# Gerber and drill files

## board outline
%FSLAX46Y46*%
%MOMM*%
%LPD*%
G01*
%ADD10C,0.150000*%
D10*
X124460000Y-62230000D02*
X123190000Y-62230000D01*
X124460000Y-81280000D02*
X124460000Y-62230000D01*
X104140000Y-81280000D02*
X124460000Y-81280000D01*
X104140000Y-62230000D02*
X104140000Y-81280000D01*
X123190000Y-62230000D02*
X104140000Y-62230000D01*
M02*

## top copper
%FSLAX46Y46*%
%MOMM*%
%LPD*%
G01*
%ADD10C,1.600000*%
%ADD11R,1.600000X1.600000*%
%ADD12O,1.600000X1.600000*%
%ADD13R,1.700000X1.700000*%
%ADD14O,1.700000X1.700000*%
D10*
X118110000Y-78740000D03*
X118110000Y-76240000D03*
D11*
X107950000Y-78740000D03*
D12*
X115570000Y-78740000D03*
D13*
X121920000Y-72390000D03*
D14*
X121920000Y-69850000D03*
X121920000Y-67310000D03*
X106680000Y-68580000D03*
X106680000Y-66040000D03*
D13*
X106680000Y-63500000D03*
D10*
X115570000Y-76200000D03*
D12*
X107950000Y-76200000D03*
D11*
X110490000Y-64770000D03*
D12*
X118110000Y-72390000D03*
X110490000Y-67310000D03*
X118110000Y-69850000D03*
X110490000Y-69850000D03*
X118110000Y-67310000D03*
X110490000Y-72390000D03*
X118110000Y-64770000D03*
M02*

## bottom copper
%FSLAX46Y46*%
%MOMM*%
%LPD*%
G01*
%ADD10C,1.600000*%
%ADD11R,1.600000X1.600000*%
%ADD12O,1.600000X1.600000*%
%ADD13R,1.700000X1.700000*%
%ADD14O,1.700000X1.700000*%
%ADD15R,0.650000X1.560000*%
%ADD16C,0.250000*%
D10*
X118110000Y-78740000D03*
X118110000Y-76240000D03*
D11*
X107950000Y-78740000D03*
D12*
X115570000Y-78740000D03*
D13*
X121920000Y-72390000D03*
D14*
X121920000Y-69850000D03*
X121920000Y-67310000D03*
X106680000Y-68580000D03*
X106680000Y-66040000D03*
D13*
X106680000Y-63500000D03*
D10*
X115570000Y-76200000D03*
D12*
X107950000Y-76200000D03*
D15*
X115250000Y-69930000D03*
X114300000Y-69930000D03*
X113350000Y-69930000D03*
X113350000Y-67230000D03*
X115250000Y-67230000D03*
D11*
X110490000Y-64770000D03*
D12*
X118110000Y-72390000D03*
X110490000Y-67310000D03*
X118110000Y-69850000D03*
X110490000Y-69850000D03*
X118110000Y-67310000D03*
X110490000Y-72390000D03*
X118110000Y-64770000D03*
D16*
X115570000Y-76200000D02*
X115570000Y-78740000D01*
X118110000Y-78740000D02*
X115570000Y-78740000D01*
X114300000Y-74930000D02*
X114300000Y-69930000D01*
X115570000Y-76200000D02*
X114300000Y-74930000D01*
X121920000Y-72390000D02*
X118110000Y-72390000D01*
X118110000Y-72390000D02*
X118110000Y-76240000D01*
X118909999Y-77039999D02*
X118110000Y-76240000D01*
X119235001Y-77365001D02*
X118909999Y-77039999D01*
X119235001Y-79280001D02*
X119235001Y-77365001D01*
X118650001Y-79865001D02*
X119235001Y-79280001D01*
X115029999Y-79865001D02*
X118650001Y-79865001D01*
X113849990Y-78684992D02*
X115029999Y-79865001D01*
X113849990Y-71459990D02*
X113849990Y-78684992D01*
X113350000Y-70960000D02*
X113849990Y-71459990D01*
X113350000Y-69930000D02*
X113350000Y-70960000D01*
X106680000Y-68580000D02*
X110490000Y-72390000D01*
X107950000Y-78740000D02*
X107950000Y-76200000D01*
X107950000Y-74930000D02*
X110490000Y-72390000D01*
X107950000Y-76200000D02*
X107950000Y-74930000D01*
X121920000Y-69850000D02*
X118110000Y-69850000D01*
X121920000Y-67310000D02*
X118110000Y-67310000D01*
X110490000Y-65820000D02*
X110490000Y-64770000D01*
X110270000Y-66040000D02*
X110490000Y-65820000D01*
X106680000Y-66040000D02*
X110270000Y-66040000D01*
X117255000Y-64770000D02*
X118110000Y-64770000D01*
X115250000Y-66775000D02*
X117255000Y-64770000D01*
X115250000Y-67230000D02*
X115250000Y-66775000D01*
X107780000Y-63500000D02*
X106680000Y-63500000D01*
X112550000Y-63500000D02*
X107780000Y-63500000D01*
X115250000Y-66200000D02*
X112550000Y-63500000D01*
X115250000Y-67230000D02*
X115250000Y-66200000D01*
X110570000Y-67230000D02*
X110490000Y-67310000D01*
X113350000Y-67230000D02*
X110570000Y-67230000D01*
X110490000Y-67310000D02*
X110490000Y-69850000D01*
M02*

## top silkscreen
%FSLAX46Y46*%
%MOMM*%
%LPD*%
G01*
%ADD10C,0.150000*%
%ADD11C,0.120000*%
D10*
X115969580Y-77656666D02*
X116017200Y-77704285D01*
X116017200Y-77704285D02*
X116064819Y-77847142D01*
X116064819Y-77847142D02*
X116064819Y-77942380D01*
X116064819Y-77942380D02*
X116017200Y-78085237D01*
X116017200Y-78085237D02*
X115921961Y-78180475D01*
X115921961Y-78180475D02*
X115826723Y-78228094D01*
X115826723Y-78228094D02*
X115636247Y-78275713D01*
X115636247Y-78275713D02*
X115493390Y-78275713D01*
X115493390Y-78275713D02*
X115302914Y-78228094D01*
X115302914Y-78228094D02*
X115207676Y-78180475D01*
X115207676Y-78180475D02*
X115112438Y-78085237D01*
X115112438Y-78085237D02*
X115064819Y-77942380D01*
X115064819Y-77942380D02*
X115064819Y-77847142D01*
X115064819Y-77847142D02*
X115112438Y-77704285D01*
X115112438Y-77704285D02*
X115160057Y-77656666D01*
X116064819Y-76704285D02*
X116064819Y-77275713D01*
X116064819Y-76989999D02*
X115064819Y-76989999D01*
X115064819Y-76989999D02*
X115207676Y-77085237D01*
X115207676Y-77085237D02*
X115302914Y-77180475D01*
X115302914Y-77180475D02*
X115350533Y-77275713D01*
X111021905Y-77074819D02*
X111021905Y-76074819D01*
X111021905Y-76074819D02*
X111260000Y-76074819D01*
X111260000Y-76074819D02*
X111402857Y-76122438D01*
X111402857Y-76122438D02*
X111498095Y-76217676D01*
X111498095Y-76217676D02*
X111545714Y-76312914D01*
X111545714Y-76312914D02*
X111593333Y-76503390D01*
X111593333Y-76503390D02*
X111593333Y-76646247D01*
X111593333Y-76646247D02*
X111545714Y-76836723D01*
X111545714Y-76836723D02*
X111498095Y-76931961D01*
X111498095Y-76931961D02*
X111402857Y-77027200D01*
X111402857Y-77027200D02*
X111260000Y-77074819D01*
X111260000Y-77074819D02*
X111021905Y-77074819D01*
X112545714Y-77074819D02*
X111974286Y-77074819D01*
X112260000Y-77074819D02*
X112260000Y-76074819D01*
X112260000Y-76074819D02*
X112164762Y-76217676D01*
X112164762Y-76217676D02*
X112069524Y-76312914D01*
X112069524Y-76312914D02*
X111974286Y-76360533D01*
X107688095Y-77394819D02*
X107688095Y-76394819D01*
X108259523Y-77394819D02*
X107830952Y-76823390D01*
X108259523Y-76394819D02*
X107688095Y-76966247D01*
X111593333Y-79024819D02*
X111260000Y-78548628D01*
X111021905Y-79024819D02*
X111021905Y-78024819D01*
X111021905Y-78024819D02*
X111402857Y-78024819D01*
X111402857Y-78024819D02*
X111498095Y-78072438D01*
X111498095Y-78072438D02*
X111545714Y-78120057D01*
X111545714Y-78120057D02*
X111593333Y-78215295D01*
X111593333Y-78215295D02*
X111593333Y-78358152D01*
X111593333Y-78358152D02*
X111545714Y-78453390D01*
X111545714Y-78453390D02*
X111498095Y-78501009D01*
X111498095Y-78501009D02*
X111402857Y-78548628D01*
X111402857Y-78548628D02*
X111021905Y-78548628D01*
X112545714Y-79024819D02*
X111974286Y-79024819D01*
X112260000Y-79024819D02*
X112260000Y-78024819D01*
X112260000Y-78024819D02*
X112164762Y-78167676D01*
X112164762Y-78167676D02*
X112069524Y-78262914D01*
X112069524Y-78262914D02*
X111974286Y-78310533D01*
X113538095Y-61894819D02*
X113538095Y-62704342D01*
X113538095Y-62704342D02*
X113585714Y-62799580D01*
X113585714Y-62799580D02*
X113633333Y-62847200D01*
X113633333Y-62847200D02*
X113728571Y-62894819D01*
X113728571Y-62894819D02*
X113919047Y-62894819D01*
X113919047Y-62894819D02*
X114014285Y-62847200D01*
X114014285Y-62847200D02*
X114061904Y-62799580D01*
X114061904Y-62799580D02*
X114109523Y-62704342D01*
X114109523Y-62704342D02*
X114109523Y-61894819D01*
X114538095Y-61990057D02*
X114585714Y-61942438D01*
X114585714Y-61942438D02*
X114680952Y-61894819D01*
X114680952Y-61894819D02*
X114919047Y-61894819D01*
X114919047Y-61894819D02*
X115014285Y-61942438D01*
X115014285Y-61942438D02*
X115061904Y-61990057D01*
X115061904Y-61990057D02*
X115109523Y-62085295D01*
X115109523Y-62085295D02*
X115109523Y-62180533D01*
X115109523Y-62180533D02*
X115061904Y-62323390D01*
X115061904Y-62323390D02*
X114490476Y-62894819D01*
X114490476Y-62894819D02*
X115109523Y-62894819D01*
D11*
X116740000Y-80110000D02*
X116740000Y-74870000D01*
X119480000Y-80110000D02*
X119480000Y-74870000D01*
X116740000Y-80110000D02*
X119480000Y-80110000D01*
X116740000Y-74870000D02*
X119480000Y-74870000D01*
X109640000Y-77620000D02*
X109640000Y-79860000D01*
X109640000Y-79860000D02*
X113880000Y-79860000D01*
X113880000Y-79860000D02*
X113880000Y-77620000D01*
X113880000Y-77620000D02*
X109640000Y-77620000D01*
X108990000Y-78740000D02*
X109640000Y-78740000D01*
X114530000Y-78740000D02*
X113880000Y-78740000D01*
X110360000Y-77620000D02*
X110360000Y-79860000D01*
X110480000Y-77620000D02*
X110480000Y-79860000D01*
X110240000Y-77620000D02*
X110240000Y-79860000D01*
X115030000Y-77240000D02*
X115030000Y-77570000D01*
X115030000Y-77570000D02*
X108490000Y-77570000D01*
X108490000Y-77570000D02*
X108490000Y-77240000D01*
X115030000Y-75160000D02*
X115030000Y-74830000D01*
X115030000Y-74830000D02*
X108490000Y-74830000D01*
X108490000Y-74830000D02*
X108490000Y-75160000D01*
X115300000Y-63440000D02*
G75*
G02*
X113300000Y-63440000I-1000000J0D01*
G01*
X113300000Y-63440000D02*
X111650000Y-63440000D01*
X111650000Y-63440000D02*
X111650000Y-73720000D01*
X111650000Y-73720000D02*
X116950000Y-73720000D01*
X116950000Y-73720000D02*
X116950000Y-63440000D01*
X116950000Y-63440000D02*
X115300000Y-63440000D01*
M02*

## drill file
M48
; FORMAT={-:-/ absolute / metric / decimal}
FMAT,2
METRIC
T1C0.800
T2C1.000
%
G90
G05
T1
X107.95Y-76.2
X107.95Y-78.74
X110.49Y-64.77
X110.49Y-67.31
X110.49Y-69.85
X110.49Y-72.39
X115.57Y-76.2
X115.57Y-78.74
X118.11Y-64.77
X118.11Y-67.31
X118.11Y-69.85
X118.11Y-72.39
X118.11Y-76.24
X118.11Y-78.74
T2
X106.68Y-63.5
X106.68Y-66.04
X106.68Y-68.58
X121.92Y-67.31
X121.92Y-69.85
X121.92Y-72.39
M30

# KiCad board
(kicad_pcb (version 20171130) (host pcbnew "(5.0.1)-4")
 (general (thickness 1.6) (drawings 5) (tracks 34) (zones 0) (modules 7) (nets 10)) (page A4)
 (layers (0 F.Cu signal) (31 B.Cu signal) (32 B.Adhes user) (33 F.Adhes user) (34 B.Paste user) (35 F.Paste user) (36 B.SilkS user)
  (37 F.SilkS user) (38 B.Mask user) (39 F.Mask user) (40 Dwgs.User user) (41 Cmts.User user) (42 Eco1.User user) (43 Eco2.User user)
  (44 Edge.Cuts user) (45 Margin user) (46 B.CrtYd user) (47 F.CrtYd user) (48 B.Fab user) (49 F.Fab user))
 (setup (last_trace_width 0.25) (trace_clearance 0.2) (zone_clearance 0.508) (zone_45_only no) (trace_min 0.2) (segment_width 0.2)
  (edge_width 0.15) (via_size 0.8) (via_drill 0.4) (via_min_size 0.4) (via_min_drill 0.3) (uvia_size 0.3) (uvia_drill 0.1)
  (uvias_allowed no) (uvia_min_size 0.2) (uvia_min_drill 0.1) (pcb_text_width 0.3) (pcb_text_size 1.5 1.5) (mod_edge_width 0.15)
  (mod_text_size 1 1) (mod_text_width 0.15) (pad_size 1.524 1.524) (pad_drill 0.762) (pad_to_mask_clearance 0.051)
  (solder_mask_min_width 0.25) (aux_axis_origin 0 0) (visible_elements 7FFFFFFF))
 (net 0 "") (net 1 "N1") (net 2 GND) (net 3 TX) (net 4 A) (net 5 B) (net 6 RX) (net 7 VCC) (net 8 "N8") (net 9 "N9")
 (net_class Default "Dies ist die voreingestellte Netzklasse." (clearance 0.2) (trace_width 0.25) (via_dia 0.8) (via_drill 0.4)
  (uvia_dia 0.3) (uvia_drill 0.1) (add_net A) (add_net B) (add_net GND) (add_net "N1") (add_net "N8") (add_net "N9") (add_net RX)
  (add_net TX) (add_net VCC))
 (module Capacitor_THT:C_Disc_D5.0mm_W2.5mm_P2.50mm (layer F.Cu) (at 118.11 78.74 90)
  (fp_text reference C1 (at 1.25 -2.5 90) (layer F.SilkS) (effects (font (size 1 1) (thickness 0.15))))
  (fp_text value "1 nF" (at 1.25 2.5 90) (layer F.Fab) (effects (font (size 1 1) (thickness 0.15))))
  (fp_line (start -1.37 -1.37) (end 3.87 -1.37) (layer F.SilkS) (width 0.12))
  (fp_line (start -1.37 1.37) (end 3.87 1.37) (layer F.SilkS) (width 0.12))
  (fp_line (start -1.37 -1.37) (end -1.37 1.37) (layer F.SilkS) (width 0.12))
  (fp_line (start 3.87 -1.37) (end 3.87 1.37) (layer F.SilkS) (width 0.12))
  (pad 1 thru_hole circle (at 0 0 90) (size 1.6 1.6) (drill 0.8) (layers *.Cu *.Mask) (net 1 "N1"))
  (pad 2 thru_hole circle (at 2.5 0 90) (size 1.6 1.6) (drill 0.8) (layers *.Cu *.Mask) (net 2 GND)))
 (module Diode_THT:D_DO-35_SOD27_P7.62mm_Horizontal (layer F.Cu) (at 107.95 78.74)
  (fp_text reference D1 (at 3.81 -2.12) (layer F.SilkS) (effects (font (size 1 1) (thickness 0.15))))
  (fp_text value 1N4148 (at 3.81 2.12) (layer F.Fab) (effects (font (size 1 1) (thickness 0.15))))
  (fp_line (start 1.69 -1.12) (end 1.69 1.12) (layer F.SilkS) (width 0.12))
  (fp_line (start 1.69 1.12) (end 5.93 1.12) (layer F.SilkS) (width 0.12))
  (fp_line (start 5.93 1.12) (end 5.93 -1.12) (layer F.SilkS) (width 0.12))
  (fp_line (start 5.93 -1.12) (end 1.69 -1.12) (layer F.SilkS) (width 0.12))
  (fp_line (start 1.04 0) (end 1.69 0) (layer F.SilkS) (width 0.12))
  (fp_line (start 6.58 0) (end 5.93 0) (layer F.SilkS) (width 0.12))
  (fp_line (start 2.41 -1.12) (end 2.41 1.12) (layer F.SilkS) (width 0.12))
  (fp_line (start 2.53 -1.12) (end 2.53 1.12) (layer F.SilkS) (width 0.12))
  (fp_line (start 2.29 -1.12) (end 2.29 1.12) (layer F.SilkS) (width 0.12))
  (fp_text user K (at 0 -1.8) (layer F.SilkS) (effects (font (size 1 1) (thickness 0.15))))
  (pad 1 thru_hole rect (at 0 0) (size 1.6 1.6) (drill 0.8) (layers *.Cu *.Mask) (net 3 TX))
  (pad 2 thru_hole oval (at 7.62 0) (size 1.6 1.6) (drill 0.8) (layers *.Cu *.Mask) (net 1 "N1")))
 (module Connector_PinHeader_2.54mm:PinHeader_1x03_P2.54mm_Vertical (layer B.Cu) (at 121.92 72.39)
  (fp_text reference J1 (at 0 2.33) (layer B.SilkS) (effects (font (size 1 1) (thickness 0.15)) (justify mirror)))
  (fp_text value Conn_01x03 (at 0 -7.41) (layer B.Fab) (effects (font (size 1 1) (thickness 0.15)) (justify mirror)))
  (pad 1 thru_hole rect (at 0 0) (size 1.7 1.7) (drill 1) (layers *.Cu *.Mask) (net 2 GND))
  (pad 2 thru_hole oval (at 0 -2.54) (size 1.7 1.7) (drill 1) (layers *.Cu *.Mask) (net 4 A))
  (pad 3 thru_hole oval (at 0 -5.08) (size 1.7 1.7) (drill 1) (layers *.Cu *.Mask) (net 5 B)))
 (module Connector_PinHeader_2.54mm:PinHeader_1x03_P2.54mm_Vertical (layer B.Cu) (at 106.68 63.5 180)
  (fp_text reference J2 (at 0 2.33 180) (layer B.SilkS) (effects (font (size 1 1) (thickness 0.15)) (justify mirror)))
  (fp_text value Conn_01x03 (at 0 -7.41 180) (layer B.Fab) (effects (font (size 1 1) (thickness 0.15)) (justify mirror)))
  (pad 3 thru_hole oval (at 0 -5.08 180) (size 1.7 1.7) (drill 1) (layers *.Cu *.Mask) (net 3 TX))
  (pad 2 thru_hole oval (at 0 -2.54 180) (size 1.7 1.7) (drill 1) (layers *.Cu *.Mask) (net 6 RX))
  (pad 1 thru_hole rect (at 0 0 180) (size 1.7 1.7) (drill 1) (layers *.Cu *.Mask) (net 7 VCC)))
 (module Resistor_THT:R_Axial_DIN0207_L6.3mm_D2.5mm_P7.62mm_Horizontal (layer F.Cu) (at 115.57 76.2 180)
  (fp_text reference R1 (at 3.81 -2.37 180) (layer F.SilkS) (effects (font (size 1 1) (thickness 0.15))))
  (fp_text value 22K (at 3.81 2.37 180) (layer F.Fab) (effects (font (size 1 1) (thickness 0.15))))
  (fp_line (start 0.54 -1.04) (end 0.54 -1.37) (layer F.SilkS) (width 0.12))
  (fp_line (start 0.54 -1.37) (end 7.08 -1.37) (layer F.SilkS) (width 0.12))
  (fp_line (start 7.08 -1.37) (end 7.08 -1.04) (layer F.SilkS) (width 0.12))
  (fp_line (start 0.54 1.04) (end 0.54 1.37) (layer F.SilkS) (width 0.12))
  (fp_line (start 0.54 1.37) (end 7.08 1.37) (layer F.SilkS) (width 0.12))
  (fp_line (start 7.08 1.37) (end 7.08 1.04) (layer F.SilkS) (width 0.12))
  (pad 1 thru_hole circle (at 0 0 180) (size 1.6 1.6) (drill 0.8) (layers *.Cu *.Mask) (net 1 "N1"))
  (pad 2 thru_hole oval (at 7.62 0 180) (size 1.6 1.6) (drill 0.8) (layers *.Cu *.Mask) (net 3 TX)))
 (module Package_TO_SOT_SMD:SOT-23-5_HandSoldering (layer B.Cu) (at 114.3 68.58 90)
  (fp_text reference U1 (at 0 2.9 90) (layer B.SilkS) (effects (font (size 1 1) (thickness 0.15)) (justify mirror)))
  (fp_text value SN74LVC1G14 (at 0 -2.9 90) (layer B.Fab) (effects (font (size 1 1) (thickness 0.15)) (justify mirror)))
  (pad 1 smd rect (at -1.35 0.95 90) (size 1.56 0.65) (layers B.Cu B.Paste B.Mask) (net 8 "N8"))
  (pad 2 smd rect (at -1.35 0 90) (size 1.56 0.65) (layers B.Cu B.Paste B.Mask) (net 1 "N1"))
  (pad 3 smd rect (at -1.35 -0.95 90) (size 1.56 0.65) (layers B.Cu B.Paste B.Mask) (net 2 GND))
  (pad 4 smd rect (at 1.35 -0.95 90) (size 1.56 0.65) (layers B.Cu B.Paste B.Mask) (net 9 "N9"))
  (pad 5 smd rect (at 1.35 0.95 90) (size 1.56 0.65) (layers B.Cu B.Paste B.Mask) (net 7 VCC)))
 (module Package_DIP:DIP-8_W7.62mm (layer F.Cu) (at 110.49 64.77)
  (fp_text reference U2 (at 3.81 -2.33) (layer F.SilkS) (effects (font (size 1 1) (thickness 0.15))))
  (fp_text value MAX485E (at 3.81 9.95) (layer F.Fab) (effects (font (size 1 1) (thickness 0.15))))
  (fp_arc (start 3.81 -1.33) (end 2.81 -1.33) (angle -180) (layer F.SilkS) (width 0.12))
  (fp_line (start 2.81 -1.33) (end 1.16 -1.33) (layer F.SilkS) (width 0.12))
  (fp_line (start 1.16 -1.33) (end 1.16 8.95) (layer F.SilkS) (width 0.12))
  (fp_line (start 1.16 8.95) (end 6.46 8.95) (layer F.SilkS) (width 0.12))
  (fp_line (start 6.46 8.95) (end 6.46 -1.33) (layer F.SilkS) (width 0.12))
  (fp_line (start 6.46 -1.33) (end 4.81 -1.33) (layer F.SilkS) (width 0.12))
  (pad 1 thru_hole rect (at 0 0) (size 1.6 1.6) (drill 0.8) (layers *.Cu *.Mask) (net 6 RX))
  (pad 5 thru_hole oval (at 7.62 7.62) (size 1.6 1.6) (drill 0.8) (layers *.Cu *.Mask) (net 2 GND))
  (pad 2 thru_hole oval (at 0 2.54) (size 1.6 1.6) (drill 0.8) (layers *.Cu *.Mask) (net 9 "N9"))
  (pad 6 thru_hole oval (at 7.62 5.08) (size 1.6 1.6) (drill 0.8) (layers *.Cu *.Mask) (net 4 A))
  (pad 3 thru_hole oval (at 0 5.08) (size 1.6 1.6) (drill 0.8) (layers *.Cu *.Mask) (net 9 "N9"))
  (pad 7 thru_hole oval (at 7.62 2.54) (size 1.6 1.6) (drill 0.8) (layers *.Cu *.Mask) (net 5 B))
  (pad 4 thru_hole oval (at 0 7.62) (size 1.6 1.6) (drill 0.8) (layers *.Cu *.Mask) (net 3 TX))
  (pad 8 thru_hole oval (at 7.62 0) (size 1.6 1.6) (drill 0.8) (layers *.Cu *.Mask) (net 7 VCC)))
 (gr_line (start 124.46 62.23) (end 123.19 62.23) (layer Edge.Cuts) (width 0.15))
 (gr_line (start 124.46 81.28) (end 124.46 62.23) (layer Edge.Cuts) (width 0.15))
 (gr_line (start 104.14 81.28) (end 124.46 81.28) (layer Edge.Cuts) (width 0.15))
 (gr_line (start 104.14 62.23) (end 104.14 81.28) (layer Edge.Cuts) (width 0.15))
 (gr_line (start 123.19 62.23) (end 104.14 62.23) (layer Edge.Cuts) (width 0.15))
 (segment (start 115.57 76.2) (end 115.57 78.74) (width 0.25) (layer B.Cu) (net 1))
 (segment (start 118.11 78.74) (end 115.57 78.74) (width 0.25) (layer B.Cu) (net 1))
 (segment (start 114.3 74.93) (end 114.3 69.93) (width 0.25) (layer B.Cu) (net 1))
 (segment (start 115.57 76.2) (end 114.3 74.93) (width 0.25) (layer B.Cu) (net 1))
 (segment (start 121.92 72.39) (end 118.11 72.39) (width 0.25) (layer B.Cu) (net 2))
 (segment (start 118.11 72.39) (end 118.11 76.24) (width 0.25) (layer B.Cu) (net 2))
 (segment (start 118.909999 77.039999) (end 118.11 76.24) (width 0.25) (layer B.Cu) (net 2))
 (segment (start 119.235001 77.365001) (end 118.909999 77.039999) (width 0.25) (layer B.Cu) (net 2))
 (segment (start 119.235001 79.280001) (end 119.235001 77.365001) (width 0.25) (layer B.Cu) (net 2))
 (segment (start 118.650001 79.865001) (end 119.235001 79.280001) (width 0.25) (layer B.Cu) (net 2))
 (segment (start 115.029999 79.865001) (end 118.650001 79.865001) (width 0.25) (layer B.Cu) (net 2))
 (segment (start 113.84999 78.684992) (end 115.029999 79.865001) (width 0.25) (layer B.Cu) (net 2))
 (segment (start 113.84999 71.45999) (end 113.84999 78.684992) (width 0.25) (layer B.Cu) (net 2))
 (segment (start 113.35 70.96) (end 113.84999 71.45999) (width 0.25) (layer B.Cu) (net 2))
 (segment (start 113.35 69.93) (end 113.35 70.96) (width 0.25) (layer B.Cu) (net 2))
 (segment (start 106.68 68.58) (end 110.49 72.39) (width 0.25) (layer B.Cu) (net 3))
 (segment (start 107.95 78.74) (end 107.95 76.2) (width 0.25) (layer B.Cu) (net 3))
 (segment (start 107.95 74.93) (end 110.49 72.39) (width 0.25) (layer B.Cu) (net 3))
 (segment (start 107.95 76.2) (end 107.95 74.93) (width 0.25) (layer B.Cu) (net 3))
 (segment (start 121.92 69.85) (end 118.11 69.85) (width 0.25) (layer B.Cu) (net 4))
 (segment (start 121.92 67.31) (end 118.11 67.31) (width 0.25) (layer B.Cu) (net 5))
 (segment (start 110.49 65.82) (end 110.49 64.77) (width 0.25) (layer B.Cu) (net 6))
 (segment (start 110.27 66.04) (end 110.49 65.82) (width 0.25) (layer B.Cu) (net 6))
 (segment (start 106.68 66.04) (end 110.27 66.04) (width 0.25) (layer B.Cu) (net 6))
 (segment (start 117.255 64.77) (end 118.11 64.77) (width 0.25) (layer B.Cu) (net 7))
 (segment (start 115.25 66.775) (end 117.255 64.77) (width 0.25) (layer B.Cu) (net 7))
 (segment (start 115.25 67.23) (end 115.25 66.775) (width 0.25) (layer B.Cu) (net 7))
 (segment (start 107.78 63.5) (end 106.68 63.5) (width 0.25) (layer B.Cu) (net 7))
 (segment (start 112.55 63.5) (end 107.78 63.5) (width 0.25) (layer B.Cu) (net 7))
 (segment (start 115.25 66.2) (end 112.55 63.5) (width 0.25) (layer B.Cu) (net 7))
 (segment (start 115.25 67.23) (end 115.25 66.2) (width 0.25) (layer B.Cu) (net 7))
 (segment (start 110.57 67.23) (end 110.49 67.31) (width 0.25) (layer B.Cu) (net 9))
 (segment (start 113.35 67.23) (end 110.57 67.23) (width 0.25) (layer B.Cu) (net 9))
 (segment (start 110.49 67.31) (end 110.49 69.85) (width 0.25) (layer B.Cu) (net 9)))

